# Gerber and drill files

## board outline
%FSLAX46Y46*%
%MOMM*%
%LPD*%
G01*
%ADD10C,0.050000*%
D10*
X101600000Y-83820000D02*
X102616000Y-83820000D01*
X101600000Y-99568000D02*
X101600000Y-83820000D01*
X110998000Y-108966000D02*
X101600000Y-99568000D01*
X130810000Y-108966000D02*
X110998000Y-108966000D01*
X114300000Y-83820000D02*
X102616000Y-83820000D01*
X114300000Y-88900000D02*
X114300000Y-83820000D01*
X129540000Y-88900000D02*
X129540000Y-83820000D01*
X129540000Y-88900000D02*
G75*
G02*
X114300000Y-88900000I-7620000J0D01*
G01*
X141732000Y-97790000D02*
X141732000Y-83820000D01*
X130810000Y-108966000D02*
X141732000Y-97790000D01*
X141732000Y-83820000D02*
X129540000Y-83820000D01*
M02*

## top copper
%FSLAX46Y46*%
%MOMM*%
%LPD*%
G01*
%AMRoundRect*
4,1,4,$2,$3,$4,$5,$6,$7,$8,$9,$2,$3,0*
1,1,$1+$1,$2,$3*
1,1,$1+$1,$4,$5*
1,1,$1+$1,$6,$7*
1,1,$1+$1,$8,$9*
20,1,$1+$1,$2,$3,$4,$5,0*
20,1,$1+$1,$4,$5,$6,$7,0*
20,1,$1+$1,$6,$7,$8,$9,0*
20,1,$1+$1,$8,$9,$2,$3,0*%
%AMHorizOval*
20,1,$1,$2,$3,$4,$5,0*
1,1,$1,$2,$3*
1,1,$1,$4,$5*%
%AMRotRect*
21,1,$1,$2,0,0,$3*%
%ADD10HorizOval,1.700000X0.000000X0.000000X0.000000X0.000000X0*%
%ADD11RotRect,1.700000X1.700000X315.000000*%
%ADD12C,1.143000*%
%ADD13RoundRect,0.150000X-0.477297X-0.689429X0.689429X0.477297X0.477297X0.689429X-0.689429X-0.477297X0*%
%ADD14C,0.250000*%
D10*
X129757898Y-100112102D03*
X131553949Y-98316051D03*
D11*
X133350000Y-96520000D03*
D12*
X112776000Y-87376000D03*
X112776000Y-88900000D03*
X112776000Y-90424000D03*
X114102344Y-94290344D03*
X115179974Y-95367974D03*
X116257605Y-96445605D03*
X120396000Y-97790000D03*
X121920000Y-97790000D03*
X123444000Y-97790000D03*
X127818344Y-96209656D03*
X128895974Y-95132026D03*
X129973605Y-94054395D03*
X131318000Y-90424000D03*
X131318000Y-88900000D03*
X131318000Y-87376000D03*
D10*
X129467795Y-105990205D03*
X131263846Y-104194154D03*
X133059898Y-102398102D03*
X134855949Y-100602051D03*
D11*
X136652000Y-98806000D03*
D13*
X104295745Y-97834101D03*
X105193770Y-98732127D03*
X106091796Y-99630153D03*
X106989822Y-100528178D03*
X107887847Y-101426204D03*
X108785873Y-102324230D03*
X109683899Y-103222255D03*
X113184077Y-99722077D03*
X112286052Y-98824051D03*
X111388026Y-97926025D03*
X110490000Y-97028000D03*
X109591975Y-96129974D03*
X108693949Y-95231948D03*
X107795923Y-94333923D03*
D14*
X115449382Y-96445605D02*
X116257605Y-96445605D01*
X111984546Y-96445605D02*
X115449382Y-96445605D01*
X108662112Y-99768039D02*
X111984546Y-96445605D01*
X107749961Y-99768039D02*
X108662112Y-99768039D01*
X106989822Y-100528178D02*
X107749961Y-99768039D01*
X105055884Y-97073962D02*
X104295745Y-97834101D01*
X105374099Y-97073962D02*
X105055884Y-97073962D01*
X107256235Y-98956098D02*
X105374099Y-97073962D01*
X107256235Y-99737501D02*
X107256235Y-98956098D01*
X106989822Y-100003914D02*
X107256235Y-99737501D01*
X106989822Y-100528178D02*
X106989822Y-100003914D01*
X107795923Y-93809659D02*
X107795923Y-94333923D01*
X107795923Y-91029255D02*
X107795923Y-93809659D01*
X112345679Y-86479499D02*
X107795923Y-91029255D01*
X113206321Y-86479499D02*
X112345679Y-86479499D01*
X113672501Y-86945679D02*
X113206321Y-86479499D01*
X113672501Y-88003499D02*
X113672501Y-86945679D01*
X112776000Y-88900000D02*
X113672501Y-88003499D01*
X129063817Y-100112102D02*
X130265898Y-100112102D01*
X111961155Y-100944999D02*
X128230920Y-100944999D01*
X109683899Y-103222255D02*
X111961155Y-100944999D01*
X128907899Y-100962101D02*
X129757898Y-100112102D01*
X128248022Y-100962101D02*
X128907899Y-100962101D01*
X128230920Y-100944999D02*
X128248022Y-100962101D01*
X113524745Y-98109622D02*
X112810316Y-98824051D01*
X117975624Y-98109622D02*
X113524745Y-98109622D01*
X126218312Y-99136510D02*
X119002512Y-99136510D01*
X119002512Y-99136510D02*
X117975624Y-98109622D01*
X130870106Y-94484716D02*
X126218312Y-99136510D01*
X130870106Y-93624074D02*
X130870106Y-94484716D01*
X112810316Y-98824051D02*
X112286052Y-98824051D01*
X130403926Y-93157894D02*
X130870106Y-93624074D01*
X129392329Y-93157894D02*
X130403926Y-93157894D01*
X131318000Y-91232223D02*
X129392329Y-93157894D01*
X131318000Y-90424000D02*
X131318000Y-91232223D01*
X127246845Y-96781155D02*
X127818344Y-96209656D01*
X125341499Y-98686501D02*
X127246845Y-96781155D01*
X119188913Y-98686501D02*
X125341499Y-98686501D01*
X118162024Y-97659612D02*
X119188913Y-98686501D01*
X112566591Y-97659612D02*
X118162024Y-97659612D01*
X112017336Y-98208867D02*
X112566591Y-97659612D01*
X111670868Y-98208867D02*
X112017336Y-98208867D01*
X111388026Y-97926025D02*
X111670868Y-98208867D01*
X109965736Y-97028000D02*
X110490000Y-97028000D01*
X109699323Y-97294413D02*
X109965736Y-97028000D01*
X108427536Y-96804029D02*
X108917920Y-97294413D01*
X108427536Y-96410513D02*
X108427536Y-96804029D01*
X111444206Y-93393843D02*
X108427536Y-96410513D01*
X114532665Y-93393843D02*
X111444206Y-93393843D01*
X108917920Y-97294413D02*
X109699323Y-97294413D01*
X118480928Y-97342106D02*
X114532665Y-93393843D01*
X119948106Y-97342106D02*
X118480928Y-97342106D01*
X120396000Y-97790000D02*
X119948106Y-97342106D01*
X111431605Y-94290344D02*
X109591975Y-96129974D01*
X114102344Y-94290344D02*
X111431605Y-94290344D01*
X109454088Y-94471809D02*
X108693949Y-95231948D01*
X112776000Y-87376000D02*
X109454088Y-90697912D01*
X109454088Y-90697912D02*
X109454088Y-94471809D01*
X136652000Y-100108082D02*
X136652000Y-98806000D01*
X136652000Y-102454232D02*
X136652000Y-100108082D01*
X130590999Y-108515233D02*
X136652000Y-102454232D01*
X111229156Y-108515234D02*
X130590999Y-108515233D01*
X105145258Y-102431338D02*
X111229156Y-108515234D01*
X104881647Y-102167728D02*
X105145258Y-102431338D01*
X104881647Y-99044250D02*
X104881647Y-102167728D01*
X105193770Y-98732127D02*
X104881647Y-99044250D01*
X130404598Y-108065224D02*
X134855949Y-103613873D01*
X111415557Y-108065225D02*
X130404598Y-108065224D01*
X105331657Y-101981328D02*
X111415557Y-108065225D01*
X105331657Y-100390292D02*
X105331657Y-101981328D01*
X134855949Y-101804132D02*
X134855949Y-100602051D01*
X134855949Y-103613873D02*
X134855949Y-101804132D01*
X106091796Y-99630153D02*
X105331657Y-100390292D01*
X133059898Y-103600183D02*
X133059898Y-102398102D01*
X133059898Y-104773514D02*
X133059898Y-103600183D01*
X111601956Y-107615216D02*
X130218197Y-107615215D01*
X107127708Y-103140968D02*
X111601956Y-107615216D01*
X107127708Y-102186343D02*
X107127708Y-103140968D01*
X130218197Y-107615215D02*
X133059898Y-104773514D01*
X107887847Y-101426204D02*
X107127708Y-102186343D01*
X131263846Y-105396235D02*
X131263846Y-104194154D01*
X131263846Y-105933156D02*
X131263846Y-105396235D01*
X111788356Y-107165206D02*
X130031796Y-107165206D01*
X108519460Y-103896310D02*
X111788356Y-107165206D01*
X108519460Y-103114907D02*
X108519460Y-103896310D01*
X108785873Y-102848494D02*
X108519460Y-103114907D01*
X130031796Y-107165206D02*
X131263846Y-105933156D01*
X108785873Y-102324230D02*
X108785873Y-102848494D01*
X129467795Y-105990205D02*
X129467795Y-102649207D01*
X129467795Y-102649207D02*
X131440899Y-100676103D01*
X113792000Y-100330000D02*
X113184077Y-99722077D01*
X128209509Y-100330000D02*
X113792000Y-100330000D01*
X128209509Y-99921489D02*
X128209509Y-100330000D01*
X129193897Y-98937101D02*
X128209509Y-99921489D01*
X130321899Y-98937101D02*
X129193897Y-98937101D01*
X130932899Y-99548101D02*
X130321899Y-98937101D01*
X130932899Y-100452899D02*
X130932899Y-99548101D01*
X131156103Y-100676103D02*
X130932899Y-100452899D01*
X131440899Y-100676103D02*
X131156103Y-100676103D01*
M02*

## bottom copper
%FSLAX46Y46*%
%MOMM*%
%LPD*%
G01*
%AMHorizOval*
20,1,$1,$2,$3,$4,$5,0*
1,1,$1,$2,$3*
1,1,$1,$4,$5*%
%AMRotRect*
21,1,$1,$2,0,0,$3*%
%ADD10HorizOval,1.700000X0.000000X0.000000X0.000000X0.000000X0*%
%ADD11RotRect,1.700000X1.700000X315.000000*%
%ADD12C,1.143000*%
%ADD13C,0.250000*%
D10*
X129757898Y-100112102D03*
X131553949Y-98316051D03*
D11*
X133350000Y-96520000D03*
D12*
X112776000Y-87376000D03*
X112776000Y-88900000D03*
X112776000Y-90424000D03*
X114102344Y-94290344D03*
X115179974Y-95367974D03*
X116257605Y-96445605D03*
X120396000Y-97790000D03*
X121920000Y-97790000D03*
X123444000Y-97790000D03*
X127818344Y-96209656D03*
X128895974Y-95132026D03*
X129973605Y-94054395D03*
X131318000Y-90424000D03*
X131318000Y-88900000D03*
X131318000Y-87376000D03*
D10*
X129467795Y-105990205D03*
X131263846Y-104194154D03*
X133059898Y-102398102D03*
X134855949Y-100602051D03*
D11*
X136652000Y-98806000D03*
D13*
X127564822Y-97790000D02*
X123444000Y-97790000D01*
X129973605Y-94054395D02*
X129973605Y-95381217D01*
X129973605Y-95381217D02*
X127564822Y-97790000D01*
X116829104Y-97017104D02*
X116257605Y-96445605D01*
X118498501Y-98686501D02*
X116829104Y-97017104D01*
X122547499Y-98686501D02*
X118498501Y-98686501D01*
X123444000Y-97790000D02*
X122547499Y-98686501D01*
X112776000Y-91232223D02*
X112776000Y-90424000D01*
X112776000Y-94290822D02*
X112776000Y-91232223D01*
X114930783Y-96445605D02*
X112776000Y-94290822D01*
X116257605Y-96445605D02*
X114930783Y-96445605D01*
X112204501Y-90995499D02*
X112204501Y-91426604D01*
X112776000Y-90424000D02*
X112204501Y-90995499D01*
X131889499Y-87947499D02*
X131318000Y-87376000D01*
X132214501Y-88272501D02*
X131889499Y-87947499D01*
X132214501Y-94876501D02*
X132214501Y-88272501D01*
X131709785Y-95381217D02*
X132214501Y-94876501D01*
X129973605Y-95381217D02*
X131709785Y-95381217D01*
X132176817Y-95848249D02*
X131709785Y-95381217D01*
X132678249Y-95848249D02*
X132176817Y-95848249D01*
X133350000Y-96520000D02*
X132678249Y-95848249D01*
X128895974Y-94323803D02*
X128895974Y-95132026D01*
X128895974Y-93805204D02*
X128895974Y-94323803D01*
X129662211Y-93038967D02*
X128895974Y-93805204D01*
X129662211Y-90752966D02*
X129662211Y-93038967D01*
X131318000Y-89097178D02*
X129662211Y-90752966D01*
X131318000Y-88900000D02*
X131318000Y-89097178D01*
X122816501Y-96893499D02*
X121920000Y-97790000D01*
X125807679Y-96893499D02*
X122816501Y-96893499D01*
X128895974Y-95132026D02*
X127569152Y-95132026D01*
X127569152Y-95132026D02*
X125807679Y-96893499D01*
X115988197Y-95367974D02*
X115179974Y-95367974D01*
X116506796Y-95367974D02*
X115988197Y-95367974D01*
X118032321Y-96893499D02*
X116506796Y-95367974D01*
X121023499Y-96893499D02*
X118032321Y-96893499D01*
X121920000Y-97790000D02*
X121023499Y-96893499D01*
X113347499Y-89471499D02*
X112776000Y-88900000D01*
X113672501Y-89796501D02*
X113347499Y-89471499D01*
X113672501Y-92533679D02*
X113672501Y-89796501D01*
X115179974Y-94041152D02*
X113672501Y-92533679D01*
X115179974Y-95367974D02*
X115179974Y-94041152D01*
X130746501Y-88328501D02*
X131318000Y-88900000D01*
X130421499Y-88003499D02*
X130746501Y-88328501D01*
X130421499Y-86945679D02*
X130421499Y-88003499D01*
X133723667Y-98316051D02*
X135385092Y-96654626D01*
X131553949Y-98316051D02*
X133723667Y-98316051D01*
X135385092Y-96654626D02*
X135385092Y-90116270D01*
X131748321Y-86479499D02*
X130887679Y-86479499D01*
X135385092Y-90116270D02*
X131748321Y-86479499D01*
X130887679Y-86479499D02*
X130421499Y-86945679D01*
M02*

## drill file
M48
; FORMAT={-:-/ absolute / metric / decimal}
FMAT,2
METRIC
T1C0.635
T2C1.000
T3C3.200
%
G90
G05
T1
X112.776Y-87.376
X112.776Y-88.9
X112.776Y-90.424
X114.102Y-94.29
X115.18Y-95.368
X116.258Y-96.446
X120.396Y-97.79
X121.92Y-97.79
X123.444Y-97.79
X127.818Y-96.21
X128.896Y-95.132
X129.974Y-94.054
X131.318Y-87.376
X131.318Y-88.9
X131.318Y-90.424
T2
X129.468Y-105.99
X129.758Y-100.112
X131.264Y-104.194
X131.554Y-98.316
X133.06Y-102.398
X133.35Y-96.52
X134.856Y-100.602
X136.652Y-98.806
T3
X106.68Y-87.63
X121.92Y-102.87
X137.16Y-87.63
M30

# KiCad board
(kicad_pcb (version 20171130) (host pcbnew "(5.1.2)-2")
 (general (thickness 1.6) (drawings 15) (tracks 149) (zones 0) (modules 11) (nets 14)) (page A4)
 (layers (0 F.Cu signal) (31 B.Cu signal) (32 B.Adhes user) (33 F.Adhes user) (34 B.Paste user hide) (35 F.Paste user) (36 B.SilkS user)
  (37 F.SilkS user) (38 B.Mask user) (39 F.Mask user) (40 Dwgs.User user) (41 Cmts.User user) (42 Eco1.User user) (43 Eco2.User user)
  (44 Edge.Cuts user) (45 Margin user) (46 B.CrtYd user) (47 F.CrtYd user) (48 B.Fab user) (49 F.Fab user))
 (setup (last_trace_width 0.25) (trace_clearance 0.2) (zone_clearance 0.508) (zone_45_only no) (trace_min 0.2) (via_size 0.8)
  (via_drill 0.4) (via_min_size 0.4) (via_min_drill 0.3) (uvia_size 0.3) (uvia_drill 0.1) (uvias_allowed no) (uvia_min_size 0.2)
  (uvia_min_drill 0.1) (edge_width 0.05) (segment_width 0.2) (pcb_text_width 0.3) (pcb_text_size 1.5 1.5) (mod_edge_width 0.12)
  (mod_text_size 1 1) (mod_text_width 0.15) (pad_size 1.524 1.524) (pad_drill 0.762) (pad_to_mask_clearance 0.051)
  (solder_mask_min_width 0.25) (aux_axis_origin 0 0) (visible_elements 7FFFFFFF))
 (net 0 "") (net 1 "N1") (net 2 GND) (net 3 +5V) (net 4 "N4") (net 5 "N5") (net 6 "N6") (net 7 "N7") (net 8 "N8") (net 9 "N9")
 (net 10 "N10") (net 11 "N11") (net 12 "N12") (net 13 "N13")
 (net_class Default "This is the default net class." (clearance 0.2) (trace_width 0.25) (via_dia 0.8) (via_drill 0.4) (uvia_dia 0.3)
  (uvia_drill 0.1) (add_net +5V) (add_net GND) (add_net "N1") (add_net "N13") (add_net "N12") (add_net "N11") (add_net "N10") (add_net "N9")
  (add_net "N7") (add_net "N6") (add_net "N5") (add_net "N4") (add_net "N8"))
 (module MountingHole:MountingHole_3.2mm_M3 (layer F.Cu) (at 121.92 102.87)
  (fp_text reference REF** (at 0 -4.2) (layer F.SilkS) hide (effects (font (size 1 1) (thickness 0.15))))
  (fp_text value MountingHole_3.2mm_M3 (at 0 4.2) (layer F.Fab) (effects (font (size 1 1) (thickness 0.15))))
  (pad 1 np_thru_hole circle (at 0 0) (size 3.2 3.2) (drill 3.2) (layers *.Cu *.Mask)))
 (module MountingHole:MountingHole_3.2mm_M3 (layer F.Cu) (at 137.16 87.63)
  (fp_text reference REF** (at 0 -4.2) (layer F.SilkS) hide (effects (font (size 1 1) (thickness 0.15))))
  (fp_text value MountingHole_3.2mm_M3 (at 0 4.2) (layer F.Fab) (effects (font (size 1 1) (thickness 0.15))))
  (pad 1 np_thru_hole circle (at 0 0) (size 3.2 3.2) (drill 3.2) (layers *.Cu *.Mask)))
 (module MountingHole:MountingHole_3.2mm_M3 (layer F.Cu) (at 106.68 87.63)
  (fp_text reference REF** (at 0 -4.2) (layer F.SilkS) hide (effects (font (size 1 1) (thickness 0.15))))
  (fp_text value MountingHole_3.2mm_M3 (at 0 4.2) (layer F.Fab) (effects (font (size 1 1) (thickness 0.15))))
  (pad 1 np_thru_hole circle (at 0 0) (size 3.2 3.2) (drill 3.2) (layers *.Cu *.Mask)))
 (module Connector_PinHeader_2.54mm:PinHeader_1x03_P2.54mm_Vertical (layer F.Cu) (at 133.35 96.52 315)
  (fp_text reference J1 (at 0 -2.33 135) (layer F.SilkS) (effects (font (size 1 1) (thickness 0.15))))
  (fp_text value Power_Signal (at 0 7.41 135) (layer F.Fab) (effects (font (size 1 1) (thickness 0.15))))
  (pad 3 thru_hole oval (at 0 5.08 315) (size 1.7 1.7) (drill 1) (layers *.Cu *.Mask) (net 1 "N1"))
  (pad 2 thru_hole oval (at 0 2.54 315) (size 1.7 1.7) (drill 1) (layers *.Cu *.Mask) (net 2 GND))
  (pad 1 thru_hole rect (at 0 0 315) (size 1.7 1.7) (drill 1) (layers *.Cu *.Mask) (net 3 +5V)))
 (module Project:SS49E (layer F.Cu) (at 112.776 90.17 90)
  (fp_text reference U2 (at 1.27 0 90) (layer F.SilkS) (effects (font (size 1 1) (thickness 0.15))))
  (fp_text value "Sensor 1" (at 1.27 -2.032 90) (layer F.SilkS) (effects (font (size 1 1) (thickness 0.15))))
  (pad 3 thru_hole circle (at 2.794 0 90) (size 1.143 1.143) (drill 0.635) (layers *.Cu *.Mask) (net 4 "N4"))
  (pad 2 thru_hole circle (at 1.27 0 90) (size 1.143 1.143) (drill 0.635) (layers *.Cu *.Mask) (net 2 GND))
  (pad 1 thru_hole circle (at -0.254 0 90) (size 1.143 1.143) (drill 0.635) (layers *.Cu *.Mask) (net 3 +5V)))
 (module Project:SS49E (layer F.Cu) (at 116.078 96.266 135)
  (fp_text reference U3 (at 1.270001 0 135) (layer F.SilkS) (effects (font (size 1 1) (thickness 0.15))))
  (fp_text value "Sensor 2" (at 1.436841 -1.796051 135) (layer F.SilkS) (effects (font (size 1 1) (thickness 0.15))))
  (pad 3 thru_hole circle (at 2.794 0 135) (size 1.143 1.143) (drill 0.635) (layers *.Cu *.Mask) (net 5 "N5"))
  (pad 2 thru_hole circle (at 1.27 0 135) (size 1.143 1.143) (drill 0.635) (layers *.Cu *.Mask) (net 2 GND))
  (pad 1 thru_hole circle (at -0.254 0 135) (size 1.143 1.143) (drill 0.635) (layers *.Cu *.Mask) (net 3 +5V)))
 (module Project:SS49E (layer F.Cu) (at 123.19 97.79 180)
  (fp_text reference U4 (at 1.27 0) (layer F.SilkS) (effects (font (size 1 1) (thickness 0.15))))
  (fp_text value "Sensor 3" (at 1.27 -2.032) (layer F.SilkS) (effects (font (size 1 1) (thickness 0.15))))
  (pad 3 thru_hole circle (at 2.794 0 180) (size 1.143 1.143) (drill 0.635) (layers *.Cu *.Mask) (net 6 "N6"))
  (pad 2 thru_hole circle (at 1.27 0 180) (size 1.143 1.143) (drill 0.635) (layers *.Cu *.Mask) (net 2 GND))
  (pad 1 thru_hole circle (at -0.254 0 180) (size 1.143 1.143) (drill 0.635) (layers *.Cu *.Mask) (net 3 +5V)))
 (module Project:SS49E (layer F.Cu) (at 129.794 94.234 225)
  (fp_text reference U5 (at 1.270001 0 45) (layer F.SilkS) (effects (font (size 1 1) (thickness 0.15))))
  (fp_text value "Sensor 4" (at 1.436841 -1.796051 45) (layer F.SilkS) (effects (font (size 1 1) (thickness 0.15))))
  (pad 3 thru_hole circle (at 2.794 0 225) (size 1.143 1.143) (drill 0.635) (layers *.Cu *.Mask) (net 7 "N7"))
  (pad 2 thru_hole circle (at 1.27 0 225) (size 1.143 1.143) (drill 0.635) (layers *.Cu *.Mask) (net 2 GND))
  (pad 1 thru_hole circle (at -0.254 0 225) (size 1.143 1.143) (drill 0.635) (layers *.Cu *.Mask) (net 3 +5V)))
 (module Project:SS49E (layer F.Cu) (at 131.318 87.63 270)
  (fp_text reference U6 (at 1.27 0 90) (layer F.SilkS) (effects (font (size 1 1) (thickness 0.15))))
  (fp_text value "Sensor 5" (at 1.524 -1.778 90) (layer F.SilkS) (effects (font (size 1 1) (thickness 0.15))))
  (pad 3 thru_hole circle (at 2.794 0 270) (size 1.143 1.143) (drill 0.635) (layers *.Cu *.Mask) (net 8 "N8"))
  (pad 2 thru_hole circle (at 1.27 0 270) (size 1.143 1.143) (drill 0.635) (layers *.Cu *.Mask) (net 2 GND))
  (pad 1 thru_hole circle (at -0.254 0 270) (size 1.143 1.143) (drill 0.635) (layers *.Cu *.Mask) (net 3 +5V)))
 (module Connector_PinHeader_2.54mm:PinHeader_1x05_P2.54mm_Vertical (layer F.Cu) (at 136.652 98.806 315)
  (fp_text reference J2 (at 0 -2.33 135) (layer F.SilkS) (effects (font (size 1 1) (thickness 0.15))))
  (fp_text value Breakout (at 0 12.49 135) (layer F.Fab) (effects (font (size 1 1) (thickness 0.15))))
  (pad 5 thru_hole oval (at 0 10.16 315) (size 1.7 1.7) (drill 1) (layers *.Cu *.Mask) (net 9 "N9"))
  (pad 4 thru_hole oval (at 0 7.62 315) (size 1.7 1.7) (drill 1) (layers *.Cu *.Mask) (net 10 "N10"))
  (pad 3 thru_hole oval (at 0 5.08 315) (size 1.7 1.7) (drill 1) (layers *.Cu *.Mask) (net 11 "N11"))
  (pad 2 thru_hole oval (at 0 2.54 315) (size 1.7 1.7) (drill 1) (layers *.Cu *.Mask) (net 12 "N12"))
  (pad 1 thru_hole rect (at 0 0 315) (size 1.7 1.7) (drill 1) (layers *.Cu *.Mask) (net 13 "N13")))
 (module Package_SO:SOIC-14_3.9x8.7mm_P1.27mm (layer F.Cu) (at 108.739911 98.778089 45)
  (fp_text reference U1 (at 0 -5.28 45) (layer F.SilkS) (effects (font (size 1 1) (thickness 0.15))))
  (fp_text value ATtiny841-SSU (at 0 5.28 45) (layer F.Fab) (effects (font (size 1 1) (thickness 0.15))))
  (pad 1 smd roundrect (at -2.475 -3.81 45) (size 1.95 0.6) (layers F.Cu F.Paste F.Mask) (roundrect_rratio 0.25) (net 3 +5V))
  (pad 2 smd roundrect (at -2.475 -2.54 45) (size 1.95 0.6) (layers F.Cu F.Paste F.Mask) (roundrect_rratio 0.25) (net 13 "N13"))
  (pad 3 smd roundrect (at -2.475 -1.27 45) (size 1.95 0.6) (layers F.Cu F.Paste F.Mask) (roundrect_rratio 0.25) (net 12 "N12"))
  (pad 4 smd roundrect (at -2.475 0 45) (size 1.95 0.6) (layers F.Cu F.Paste F.Mask) (roundrect_rratio 0.25) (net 3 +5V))
  (pad 5 smd roundrect (at -2.475 1.27 45) (size 1.95 0.6) (layers F.Cu F.Paste F.Mask) (roundrect_rratio 0.25) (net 11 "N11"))
  (pad 6 smd roundrect (at -2.475 2.54 45) (size 1.95 0.6) (layers F.Cu F.Paste F.Mask) (roundrect_rratio 0.25) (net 10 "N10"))
  (pad 7 smd roundrect (at -2.475 3.81 45) (size 1.95 0.6) (layers F.Cu F.Paste F.Mask) (roundrect_rratio 0.25) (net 1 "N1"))
  (pad 8 smd roundrect (at 2.475 3.81 45) (size 1.95 0.6) (layers F.Cu F.Paste F.Mask) (roundrect_rratio 0.25) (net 9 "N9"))
  (pad 9 smd roundrect (at 2.475 2.54 45) (size 1.95 0.6) (layers F.Cu F.Paste F.Mask) (roundrect_rratio 0.25) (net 8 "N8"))
  (pad 10 smd roundrect (at 2.475 1.27 45) (size 1.95 0.6) (layers F.Cu F.Paste F.Mask) (roundrect_rratio 0.25) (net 7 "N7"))
  (pad 11 smd roundrect (at 2.475 0 45) (size 1.95 0.6) (layers F.Cu F.Paste F.Mask) (roundrect_rratio 0.25) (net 6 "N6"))
  (pad 12 smd roundrect (at 2.475 -1.27 45) (size 1.95 0.6) (layers F.Cu F.Paste F.Mask) (roundrect_rratio 0.25) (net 5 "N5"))
  (pad 13 smd roundrect (at 2.475 -2.54 45) (size 1.95 0.6) (layers F.Cu F.Paste F.Mask) (roundrect_rratio 0.25) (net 4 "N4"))
  (pad 14 smd roundrect (at 2.475 -3.81 45) (size 1.95 0.6) (layers F.Cu F.Paste F.Mask) (roundrect_rratio 0.25) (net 2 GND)))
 (gr_line (start 101.6 83.82) (end 102.616 83.82) (layer Edge.Cuts) (width 0.05))
 (gr_line (start 101.6 99.568) (end 101.6 83.82) (layer Edge.Cuts) (width 0.05))
 (gr_line (start 110.998 108.966) (end 101.6 99.568) (layer Edge.Cuts) (width 0.05))
 (gr_line (start 130.81 108.966) (end 110.998 108.966) (layer Edge.Cuts) (width 0.05))
 (gr_line (start 114.3 83.82) (end 102.616 83.82) (layer Edge.Cuts) (width 0.05))
 (gr_line (start 114.3 88.9) (end 114.3 83.82) (layer Edge.Cuts) (width 0.05))
 (gr_line (start 129.54 88.9) (end 129.54 83.82) (layer Edge.Cuts) (width 0.05))
 (gr_arc (start 121.92 88.9) (end 114.3 88.9) (angle -180) (layer Edge.Cuts) (width 0.05))
 (gr_line (start 141.732 97.79) (end 141.732 83.82) (layer Edge.Cuts) (width 0.05))
 (gr_line (start 130.81 108.966) (end 141.732 97.79) (layer Edge.Cuts) (width 0.05))
 (gr_line (start 141.732 83.82) (end 129.54 83.82) (layer Edge.Cuts) (width 0.05))
 (segment (start 127.564822 97.79) (end 123.444 97.79) (width 0.25) (layer B.Cu) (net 3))
 (segment (start 129.973605 94.054395) (end 129.973605 95.381217) (width 0.25) (layer B.Cu) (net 3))
 (segment (start 129.973605 95.381217) (end 127.564822 97.79) (width 0.25) (layer B.Cu) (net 3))
 (segment (start 116.829104 97.017104) (end 116.257605 96.445605) (width 0.25) (layer B.Cu) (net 3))
 (segment (start 118.498501 98.686501) (end 116.829104 97.017104) (width 0.25) (layer B.Cu) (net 3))
 (segment (start 122.547499 98.686501) (end 118.498501 98.686501) (width 0.25) (layer B.Cu) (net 3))
 (segment (start 123.444 97.79) (end 122.547499 98.686501) (width 0.25) (layer B.Cu) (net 3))
 (segment (start 112.776 91.232223) (end 112.776 90.424) (width 0.25) (layer B.Cu) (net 3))
 (segment (start 112.776 94.290822) (end 112.776 91.232223) (width 0.25) (layer B.Cu) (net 3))
 (segment (start 114.930783 96.445605) (end 112.776 94.290822) (width 0.25) (layer B.Cu) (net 3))
 (segment (start 116.257605 96.445605) (end 114.930783 96.445605) (width 0.25) (layer B.Cu) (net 3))
 (segment (start 112.204501 90.995499) (end 112.204501 91.426604) (width 0.25) (layer B.Cu) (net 3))
 (segment (start 112.776 90.424) (end 112.204501 90.995499) (width 0.25) (layer B.Cu) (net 3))
 (segment (start 131.889499 87.947499) (end 131.318 87.376) (width 0.25) (layer B.Cu) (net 3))
 (segment (start 132.214501 88.272501) (end 131.889499 87.947499) (width 0.25) (layer B.Cu) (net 3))
 (segment (start 132.214501 94.876501) (end 132.214501 88.272501) (width 0.25) (layer B.Cu) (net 3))
 (segment (start 131.709785 95.381217) (end 132.214501 94.876501) (width 0.25) (layer B.Cu) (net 3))
 (segment (start 129.973605 95.381217) (end 131.709785 95.381217) (width 0.25) (layer B.Cu) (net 3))
 (segment (start 115.449382 96.445605) (end 116.257605 96.445605) (width 0.25) (layer F.Cu) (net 3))
 (segment (start 111.984546 96.445605) (end 115.449382 96.445605) (width 0.25) (layer F.Cu) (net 3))
 (segment (start 108.662112 99.768039) (end 111.984546 96.445605) (width 0.25) (layer F.Cu) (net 3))
 (segment (start 107.749961 99.768039) (end 108.662112 99.768039) (width 0.25) (layer F.Cu) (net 3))
 (segment (start 106.989822 100.528178) (end 107.749961 99.768039) (width 0.25) (layer F.Cu) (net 3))
 (segment (start 105.055884 97.073962) (end 104.295745 97.834101) (width 0.25) (layer F.Cu) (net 3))
 (segment (start 105.374099 97.073962) (end 105.055884 97.073962) (width 0.25) (layer F.Cu) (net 3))
 (segment (start 107.256235 98.956098) (end 105.374099 97.073962) (width 0.25) (layer F.Cu) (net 3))
 (segment (start 107.256235 99.737501) (end 107.256235 98.956098) (width 0.25) (layer F.Cu) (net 3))
 (segment (start 106.989822 100.003914) (end 107.256235 99.737501) (width 0.25) (layer F.Cu) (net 3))
 (segment (start 106.989822 100.528178) (end 106.989822 100.003914) (width 0.25) (layer F.Cu) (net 3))
 (segment (start 132.176817 95.848249) (end 131.709785 95.381217) (width 0.25) (layer B.Cu) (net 3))
 (segment (start 132.678249 95.848249) (end 132.176817 95.848249) (width 0.25) (layer B.Cu) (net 3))
 (segment (start 133.35 96.52) (end 132.678249 95.848249) (width 0.25) (layer B.Cu) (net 3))
 (segment (start 128.895974 94.323803) (end 128.895974 95.132026) (width 0.25) (layer B.Cu) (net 2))
 (segment (start 128.895974 93.805204) (end 128.895974 94.323803) (width 0.25) (layer B.Cu) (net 2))
 (segment (start 129.662211 93.038967) (end 128.895974 93.805204) (width 0.25) (layer B.Cu) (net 2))
 (segment (start 129.662211 90.752966) (end 129.662211 93.038967) (width 0.25) (layer B.Cu) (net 2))
 (segment (start 131.318 89.097178) (end 129.662211 90.752966) (width 0.25) (layer B.Cu) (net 2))
 (segment (start 131.318 88.9) (end 131.318 89.097178) (width 0.25) (layer B.Cu) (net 2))
 (segment (start 122.816501 96.893499) (end 121.92 97.79) (width 0.25) (layer B.Cu) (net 2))
 (segment (start 125.807679 96.893499) (end 122.816501 96.893499) (width 0.25) (layer B.Cu) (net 2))
 (segment (start 128.895974 95.132026) (end 127.569152 95.132026) (width 0.25) (layer B.Cu) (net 2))
 (segment (start 127.569152 95.132026) (end 125.807679 96.893499) (width 0.25) (layer B.Cu) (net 2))
 (segment (start 115.988197 95.367974) (end 115.179974 95.367974) (width 0.25) (layer B.Cu) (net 2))
 (segment (start 116.506796 95.367974) (end 115.988197 95.367974) (width 0.25) (layer B.Cu) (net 2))
 (segment (start 118.032321 96.893499) (end 116.506796 95.367974) (width 0.25) (layer B.Cu) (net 2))
 (segment (start 121.023499 96.893499) (end 118.032321 96.893499) (width 0.25) (layer B.Cu) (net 2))
 (segment (start 121.92 97.79) (end 121.023499 96.893499) (width 0.25) (layer B.Cu) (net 2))
 (segment (start 113.347499 89.471499) (end 112.776 88.9) (width 0.25) (layer B.Cu) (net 2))
 (segment (start 113.672501 89.796501) (end 113.347499 89.471499) (width 0.25) (layer B.Cu) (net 2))
 (segment (start 113.672501 92.533679) (end 113.672501 89.796501) (width 0.25) (layer B.Cu) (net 2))
 (segment (start 115.179974 94.041152) (end 113.672501 92.533679) (width 0.25) (layer B.Cu) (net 2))
 (segment (start 115.179974 95.367974) (end 115.179974 94.041152) (width 0.25) (layer B.Cu) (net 2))
 (segment (start 107.795923 93.809659) (end 107.795923 94.333923) (width 0.25) (layer F.Cu) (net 2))
 (segment (start 107.795923 91.029255) (end 107.795923 93.809659) (width 0.25) (layer F.Cu) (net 2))
 (segment (start 112.345679 86.479499) (end 107.795923 91.029255) (width 0.25) (layer F.Cu) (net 2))
 (segment (start 113.206321 86.479499) (end 112.345679 86.479499) (width 0.25) (layer F.Cu) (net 2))
 (segment (start 113.672501 86.945679) (end 113.206321 86.479499) (width 0.25) (layer F.Cu) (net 2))
 (segment (start 113.672501 88.003499) (end 113.672501 86.945679) (width 0.25) (layer F.Cu) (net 2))
 (segment (start 112.776 88.9) (end 113.672501 88.003499) (width 0.25) (layer F.Cu) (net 2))
 (segment (start 130.746501 88.328501) (end 131.318 88.9) (width 0.25) (layer B.Cu) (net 2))
 (segment (start 130.421499 88.003499) (end 130.746501 88.328501) (width 0.25) (layer B.Cu) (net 2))
 (segment (start 130.421499 86.945679) (end 130.421499 88.003499) (width 0.25) (layer B.Cu) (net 2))
 (segment (start 133.723667 98.316051) (end 135.385092 96.654626) (width 0.25) (layer B.Cu) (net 2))
 (segment (start 131.553949 98.316051) (end 133.723667 98.316051) (width 0.25) (layer B.Cu) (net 2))
 (segment (start 135.385092 96.654626) (end 135.385092 90.11627) (width 0.25) (layer B.Cu) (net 2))
 (segment (start 131.748321 86.479499) (end 130.887679 86.479499) (width 0.25) (layer B.Cu) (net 2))
 (segment (start 135.385092 90.11627) (end 131.748321 86.479499) (width 0.25) (layer B.Cu) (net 2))
 (segment (start 130.887679 86.479499) (end 130.421499 86.945679) (width 0.25) (layer B.Cu) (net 2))
 (segment (start 129.063817 100.112102) (end 130.265898 100.112102) (width 0.25) (layer F.Cu) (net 1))
 (segment (start 111.961155 100.944999) (end 128.23092 100.944999) (width 0.25) (layer F.Cu) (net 1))
 (segment (start 109.683899 103.222255) (end 111.961155 100.944999) (width 0.25) (layer F.Cu) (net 1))
 (segment (start 128.907899 100.962101) (end 129.757898 100.112102) (width 0.25) (layer F.Cu) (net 1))
 (segment (start 128.248022 100.962101) (end 128.907899 100.962101) (width 0.25) (layer F.Cu) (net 1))
 (segment (start 128.23092 100.944999) (end 128.248022 100.962101) (width 0.25) (layer F.Cu) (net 1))
 (segment (start 113.524745 98.109622) (end 112.810316 98.824051) (width 0.25) (layer F.Cu) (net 8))
 (segment (start 117.975624 98.109622) (end 113.524745 98.109622) (width 0.25) (layer F.Cu) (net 8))
 (segment (start 126.218312 99.13651) (end 119.002512 99.13651) (width 0.25) (layer F.Cu) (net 8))
 (segment (start 119.002512 99.13651) (end 117.975624 98.109622) (width 0.25) (layer F.Cu) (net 8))
 (segment (start 130.870106 94.484716) (end 126.218312 99.13651) (width 0.25) (layer F.Cu) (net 8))
 (segment (start 130.870106 93.624074) (end 130.870106 94.484716) (width 0.25) (layer F.Cu) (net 8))
 (segment (start 112.810316 98.824051) (end 112.286052 98.824051) (width 0.25) (layer F.Cu) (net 8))
 (segment (start 130.403926 93.157894) (end 130.870106 93.624074) (width 0.25) (layer F.Cu) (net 8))
 (segment (start 129.392329 93.157894) (end 130.403926 93.157894) (width 0.25) (layer F.Cu) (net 8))
 (segment (start 131.318 91.232223) (end 129.392329 93.157894) (width 0.25) (layer F.Cu) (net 8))
 (segment (start 131.318 90.424) (end 131.318 91.232223) (width 0.25) (layer F.Cu) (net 8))
 (segment (start 127.246845 96.781155) (end 127.818344 96.209656) (width 0.25) (layer F.Cu) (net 7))
 (segment (start 125.341499 98.686501) (end 127.246845 96.781155) (width 0.25) (layer F.Cu) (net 7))
 (segment (start 119.188913 98.686501) (end 125.341499 98.686501) (width 0.25) (layer F.Cu) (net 7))
 (segment (start 118.162024 97.659612) (end 119.188913 98.686501) (width 0.25) (layer F.Cu) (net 7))
 (segment (start 112.566591 97.659612) (end 118.162024 97.659612) (width 0.25) (layer F.Cu) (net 7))
 (segment (start 112.017336 98.208867) (end 112.566591 97.659612) (width 0.25) (layer F.Cu) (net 7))
 (segment (start 111.670868 98.208867) (end 112.017336 98.208867) (width 0.25) (layer F.Cu) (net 7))
 (segment (start 111.388026 97.926025) (end 111.670868 98.208867) (width 0.25) (layer F.Cu) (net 7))
 (segment (start 109.965736 97.028) (end 110.49 97.028) (width 0.25) (layer F.Cu) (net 6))
 (segment (start 109.699323 97.294413) (end 109.965736 97.028) (width 0.25) (layer F.Cu) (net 6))
 (segment (start 108.427536 96.804029) (end 108.91792 97.294413) (width 0.25) (layer F.Cu) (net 6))
 (segment (start 108.427536 96.410513) (end 108.427536 96.804029) (width 0.25) (layer F.Cu) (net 6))
 (segment (start 111.444206 93.393843) (end 108.427536 96.410513) (width 0.25) (layer F.Cu) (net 6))
 (segment (start 114.532665 93.393843) (end 111.444206 93.393843) (width 0.25) (layer F.Cu) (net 6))
 (segment (start 108.91792 97.294413) (end 109.699323 97.294413) (width 0.25) (layer F.Cu) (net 6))
 (segment (start 118.480928 97.342106) (end 114.532665 93.393843) (width 0.25) (layer F.Cu) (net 6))
 (segment (start 119.948106 97.342106) (end 118.480928 97.342106) (width 0.25) (layer F.Cu) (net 6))
 (segment (start 120.396 97.79) (end 119.948106 97.342106) (width 0.25) (layer F.Cu) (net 6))
 (segment (start 111.431605 94.290344) (end 109.591975 96.129974) (width 0.25) (layer F.Cu) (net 5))
 (segment (start 114.102344 94.290344) (end 111.431605 94.290344) (width 0.25) (layer F.Cu) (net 5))
 (segment (start 109.454088 94.471809) (end 108.693949 95.231948) (width 0.25) (layer F.Cu) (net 4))
 (segment (start 112.776 87.376) (end 109.454088 90.697912) (width 0.25) (layer F.Cu) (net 4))
 (segment (start 109.454088 90.697912) (end 109.454088 94.471809) (width 0.25) (layer F.Cu) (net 4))
 (segment (start 136.652 100.108082) (end 136.652 98.806) (width 0.25) (layer F.Cu) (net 13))
 (segment (start 136.652 102.454232) (end 136.652 100.108082) (width 0.25) (layer F.Cu) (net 13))
 (segment (start 130.590999 108.515233) (end 136.652 102.454232) (width 0.25) (layer F.Cu) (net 13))
 (segment (start 111.229156 108.515234) (end 130.590999 108.515233) (width 0.25) (layer F.Cu) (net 13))
 (segment (start 105.145258 102.431338) (end 111.229156 108.515234) (width 0.25) (layer F.Cu) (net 13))
 (segment (start 104.881647 102.167728) (end 105.145258 102.431338) (width 0.25) (layer F.Cu) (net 13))
 (segment (start 104.881647 99.04425) (end 104.881647 102.167728) (width 0.25) (layer F.Cu) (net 13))
 (segment (start 105.19377 98.732127) (end 104.881647 99.04425) (width 0.25) (layer F.Cu) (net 13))
 (segment (start 130.404598 108.065224) (end 134.855949 103.613873) (width 0.25) (layer F.Cu) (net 12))
 (segment (start 111.415557 108.065225) (end 130.404598 108.065224) (width 0.25) (layer F.Cu) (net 12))
 (segment (start 105.331657 101.981328) (end 111.415557 108.065225) (width 0.25) (layer F.Cu) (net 12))
 (segment (start 105.331657 100.390292) (end 105.331657 101.981328) (width 0.25) (layer F.Cu) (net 12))
 (segment (start 134.855949 101.804132) (end 134.855949 100.602051) (width 0.25) (layer F.Cu) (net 12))
 (segment (start 134.855949 103.613873) (end 134.855949 101.804132) (width 0.25) (layer F.Cu) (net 12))
 (segment (start 106.091796 99.630153) (end 105.331657 100.390292) (width 0.25) (layer F.Cu) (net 12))
 (segment (start 133.059898 103.600183) (end 133.059898 102.398102) (width 0.25) (layer F.Cu) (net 11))
 (segment (start 133.059898 104.773514) (end 133.059898 103.600183) (width 0.25) (layer F.Cu) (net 11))
 (segment (start 111.601956 107.615216) (end 130.218197 107.615215) (width 0.25) (layer F.Cu) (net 11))
 (segment (start 107.127708 103.140968) (end 111.601956 107.615216) (width 0.25) (layer F.Cu) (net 11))
 (segment (start 107.127708 102.186343) (end 107.127708 103.140968) (width 0.25) (layer F.Cu) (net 11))
 (segment (start 130.218197 107.615215) (end 133.059898 104.773514) (width 0.25) (layer F.Cu) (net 11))
 (segment (start 107.887847 101.426204) (end 107.127708 102.186343) (width 0.25) (layer F.Cu) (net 11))
 (segment (start 131.263846 105.396235) (end 131.263846 104.194154) (width 0.25) (layer F.Cu) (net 10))
 (segment (start 131.263846 105.933156) (end 131.263846 105.396235) (width 0.25) (layer F.Cu) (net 10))
 (segment (start 111.788356 107.165206) (end 130.031796 107.165206) (width 0.25) (layer F.Cu) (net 10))
 (segment (start 108.51946 103.89631) (end 111.788356 107.165206) (width 0.25) (layer F.Cu) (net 10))
 (segment (start 108.51946 103.114907) (end 108.51946 103.89631) (width 0.25) (layer F.Cu) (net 10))
 (segment (start 108.785873 102.848494) (end 108.51946 103.114907) (width 0.25) (layer F.Cu) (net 10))
 (segment (start 130.031796 107.165206) (end 131.263846 105.933156) (width 0.25) (layer F.Cu) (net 10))
 (segment (start 108.785873 102.32423) (end 108.785873 102.848494) (width 0.25) (layer F.Cu) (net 10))
 (segment (start 129.467795 105.990205) (end 129.467795 102.649207) (width 0.25) (layer F.Cu) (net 9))
 (segment (start 129.467795 102.649207) (end 131.440899 100.676103) (width 0.25) (layer F.Cu) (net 9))
 (segment (start 113.792 100.33) (end 113.184077 99.722077) (width 0.25) (layer F.Cu) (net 9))
 (segment (start 128.209509 100.33) (end 113.792 100.33) (width 0.25) (layer F.Cu) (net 9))
 (segment (start 128.209509 99.921489) (end 128.209509 100.33) (width 0.25) (layer F.Cu) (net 9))
 (segment (start 129.193897 98.937101) (end 128.209509 99.921489) (width 0.25) (layer F.Cu) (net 9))
 (segment (start 130.321899 98.937101) (end 129.193897 98.937101) (width 0.25) (layer F.Cu) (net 9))
 (segment (start 130.932899 99.548101) (end 130.321899 98.937101) (width 0.25) (layer F.Cu) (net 9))
 (segment (start 130.932899 100.452899) (end 130.932899 99.548101) (width 0.25) (layer F.Cu) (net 9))
 (segment (start 131.156103 100.676103) (end 130.932899 100.452899) (width 0.25) (layer F.Cu) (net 9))
 (segment (start 131.440899 100.676103) (end 131.156103 100.676103) (width 0.25) (layer F.Cu) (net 9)))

